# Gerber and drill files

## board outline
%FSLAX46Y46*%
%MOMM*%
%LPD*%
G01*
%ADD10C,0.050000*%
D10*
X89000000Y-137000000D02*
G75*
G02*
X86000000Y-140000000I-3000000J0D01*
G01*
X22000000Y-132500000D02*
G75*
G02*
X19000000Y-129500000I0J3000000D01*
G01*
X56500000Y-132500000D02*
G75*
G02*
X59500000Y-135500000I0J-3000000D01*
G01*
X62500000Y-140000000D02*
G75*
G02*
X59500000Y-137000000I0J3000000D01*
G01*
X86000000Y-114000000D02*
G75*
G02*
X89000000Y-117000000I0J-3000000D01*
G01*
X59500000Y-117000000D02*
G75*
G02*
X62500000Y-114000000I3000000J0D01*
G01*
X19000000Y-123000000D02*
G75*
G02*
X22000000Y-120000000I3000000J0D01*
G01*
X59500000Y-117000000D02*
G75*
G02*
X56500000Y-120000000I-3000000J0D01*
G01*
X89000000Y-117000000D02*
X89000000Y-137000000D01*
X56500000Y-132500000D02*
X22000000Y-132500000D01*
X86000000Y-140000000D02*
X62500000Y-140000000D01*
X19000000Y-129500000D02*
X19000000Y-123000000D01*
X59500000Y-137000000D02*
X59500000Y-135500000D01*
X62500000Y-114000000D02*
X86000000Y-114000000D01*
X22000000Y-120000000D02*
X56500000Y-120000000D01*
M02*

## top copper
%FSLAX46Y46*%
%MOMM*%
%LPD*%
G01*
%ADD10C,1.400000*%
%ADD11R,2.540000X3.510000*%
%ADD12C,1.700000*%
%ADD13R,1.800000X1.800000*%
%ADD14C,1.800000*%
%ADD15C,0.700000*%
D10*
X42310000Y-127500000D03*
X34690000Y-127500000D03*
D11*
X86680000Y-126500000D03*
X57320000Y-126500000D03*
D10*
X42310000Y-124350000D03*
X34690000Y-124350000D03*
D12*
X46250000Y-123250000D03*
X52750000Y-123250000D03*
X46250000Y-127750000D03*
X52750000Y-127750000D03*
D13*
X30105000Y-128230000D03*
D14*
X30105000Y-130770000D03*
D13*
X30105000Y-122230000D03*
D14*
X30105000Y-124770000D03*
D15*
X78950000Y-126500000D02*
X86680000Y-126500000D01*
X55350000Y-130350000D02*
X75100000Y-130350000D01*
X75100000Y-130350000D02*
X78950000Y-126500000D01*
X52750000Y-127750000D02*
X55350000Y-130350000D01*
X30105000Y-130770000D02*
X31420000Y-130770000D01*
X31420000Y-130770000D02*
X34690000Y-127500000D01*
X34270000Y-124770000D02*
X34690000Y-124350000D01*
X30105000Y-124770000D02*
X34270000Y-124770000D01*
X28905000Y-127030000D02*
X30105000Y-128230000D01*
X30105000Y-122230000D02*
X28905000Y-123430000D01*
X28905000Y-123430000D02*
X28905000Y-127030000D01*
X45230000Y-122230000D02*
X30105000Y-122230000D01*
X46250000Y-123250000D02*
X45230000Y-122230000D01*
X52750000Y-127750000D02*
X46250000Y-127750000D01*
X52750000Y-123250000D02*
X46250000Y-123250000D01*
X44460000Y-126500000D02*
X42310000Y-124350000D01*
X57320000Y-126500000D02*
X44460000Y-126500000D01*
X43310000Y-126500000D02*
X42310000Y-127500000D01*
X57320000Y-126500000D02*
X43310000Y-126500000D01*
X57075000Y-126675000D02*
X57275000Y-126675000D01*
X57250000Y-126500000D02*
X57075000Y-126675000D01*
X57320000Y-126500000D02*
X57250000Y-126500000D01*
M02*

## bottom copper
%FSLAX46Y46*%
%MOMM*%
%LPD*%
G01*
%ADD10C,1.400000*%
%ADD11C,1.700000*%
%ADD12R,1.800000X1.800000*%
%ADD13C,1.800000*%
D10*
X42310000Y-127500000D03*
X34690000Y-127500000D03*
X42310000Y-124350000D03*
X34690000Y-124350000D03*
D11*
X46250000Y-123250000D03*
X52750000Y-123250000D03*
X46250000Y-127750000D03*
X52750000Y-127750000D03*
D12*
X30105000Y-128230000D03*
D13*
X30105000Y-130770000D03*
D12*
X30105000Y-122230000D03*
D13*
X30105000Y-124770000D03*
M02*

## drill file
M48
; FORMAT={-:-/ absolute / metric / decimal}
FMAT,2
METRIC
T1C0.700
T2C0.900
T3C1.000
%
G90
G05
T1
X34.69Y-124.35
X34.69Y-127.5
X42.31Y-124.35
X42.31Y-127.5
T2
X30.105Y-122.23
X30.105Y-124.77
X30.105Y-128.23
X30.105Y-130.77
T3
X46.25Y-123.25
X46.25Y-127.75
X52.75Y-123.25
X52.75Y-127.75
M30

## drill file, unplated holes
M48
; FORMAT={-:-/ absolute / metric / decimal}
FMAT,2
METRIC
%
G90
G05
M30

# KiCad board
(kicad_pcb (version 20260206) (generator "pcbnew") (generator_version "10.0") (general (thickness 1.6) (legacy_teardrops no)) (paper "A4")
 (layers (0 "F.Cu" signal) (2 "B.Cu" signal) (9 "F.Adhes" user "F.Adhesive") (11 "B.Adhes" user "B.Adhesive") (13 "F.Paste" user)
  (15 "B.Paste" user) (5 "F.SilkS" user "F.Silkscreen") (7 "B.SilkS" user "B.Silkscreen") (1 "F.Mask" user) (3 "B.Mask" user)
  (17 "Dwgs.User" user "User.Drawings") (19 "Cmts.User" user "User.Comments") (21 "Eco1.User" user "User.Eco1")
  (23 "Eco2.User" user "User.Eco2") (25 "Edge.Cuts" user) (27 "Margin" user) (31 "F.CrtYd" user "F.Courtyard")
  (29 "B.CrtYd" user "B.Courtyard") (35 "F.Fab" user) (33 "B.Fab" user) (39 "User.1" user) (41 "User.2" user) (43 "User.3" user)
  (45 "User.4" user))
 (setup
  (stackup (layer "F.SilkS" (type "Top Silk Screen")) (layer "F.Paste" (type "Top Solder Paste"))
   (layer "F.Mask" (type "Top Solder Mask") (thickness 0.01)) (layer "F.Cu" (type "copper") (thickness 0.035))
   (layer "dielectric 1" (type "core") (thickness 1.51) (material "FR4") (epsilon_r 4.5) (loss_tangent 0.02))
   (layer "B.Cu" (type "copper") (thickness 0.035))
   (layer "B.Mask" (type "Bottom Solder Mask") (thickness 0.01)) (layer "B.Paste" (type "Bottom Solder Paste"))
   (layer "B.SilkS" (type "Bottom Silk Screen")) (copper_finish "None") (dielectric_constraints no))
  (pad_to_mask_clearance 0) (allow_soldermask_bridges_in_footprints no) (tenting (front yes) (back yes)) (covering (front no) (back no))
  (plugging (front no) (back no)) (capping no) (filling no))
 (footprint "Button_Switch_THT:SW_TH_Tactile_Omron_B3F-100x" (layer "F.Cu") (at 46.25 123.25)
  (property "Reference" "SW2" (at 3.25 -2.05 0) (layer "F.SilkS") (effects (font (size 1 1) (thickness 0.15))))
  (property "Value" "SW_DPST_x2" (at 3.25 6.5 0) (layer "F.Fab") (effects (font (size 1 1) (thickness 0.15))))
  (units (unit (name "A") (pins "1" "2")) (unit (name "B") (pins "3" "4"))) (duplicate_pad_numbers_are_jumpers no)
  (pad "1" thru_hole circle (at 0 0) (size 1.7 1.7) (drill 1) (layers "*.Cu" "*.Mask") (remove_unused_layers no) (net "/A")
   (thermal_bridge_angle 90))
  (pad "1" thru_hole circle (at 6.5 0) (size 1.7 1.7) (drill 1) (layers "*.Cu" "*.Mask") (remove_unused_layers no) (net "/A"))
  (pad "2" thru_hole circle (at 0 4.5) (size 1.7 1.7) (drill 1) (layers "*.Cu" "*.Mask") (remove_unused_layers no) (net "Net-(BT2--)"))
  (pad "2" thru_hole circle (at 6.5 4.5) (size 1.7 1.7) (drill 1) (layers "*.Cu" "*.Mask") (remove_unused_layers no) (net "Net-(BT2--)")))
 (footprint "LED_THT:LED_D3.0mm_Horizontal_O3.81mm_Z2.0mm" (layer "F.Cu") (at 30.105 122.23 -90)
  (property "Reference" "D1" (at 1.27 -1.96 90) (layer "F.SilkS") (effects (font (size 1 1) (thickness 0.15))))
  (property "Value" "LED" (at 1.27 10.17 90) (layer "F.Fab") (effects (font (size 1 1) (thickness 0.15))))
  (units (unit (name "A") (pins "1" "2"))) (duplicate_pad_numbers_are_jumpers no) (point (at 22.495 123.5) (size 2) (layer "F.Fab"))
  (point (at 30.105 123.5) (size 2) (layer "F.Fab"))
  (pad "1" thru_hole rect (at 0 0 270) (size 1.8 1.8) (drill 0.9) (layers "*.Cu" "*.Mask") (remove_unused_layers no) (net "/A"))
  (pad "2" thru_hole circle (at 2.54 0 270) (size 1.8 1.8) (drill 0.9) (layers "*.Cu" "*.Mask") (remove_unused_layers no) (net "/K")))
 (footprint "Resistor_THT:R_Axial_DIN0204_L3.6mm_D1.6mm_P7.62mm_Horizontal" (layer "F.Cu") (at 42.31 127.5 180)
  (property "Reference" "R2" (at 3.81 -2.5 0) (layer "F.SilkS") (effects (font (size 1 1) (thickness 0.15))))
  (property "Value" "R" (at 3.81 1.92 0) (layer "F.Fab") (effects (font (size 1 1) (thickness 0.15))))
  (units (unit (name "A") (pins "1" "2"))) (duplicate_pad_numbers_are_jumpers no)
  (pad "1" thru_hole circle (at 0 0 180) (size 1.4 1.4) (drill 0.7) (layers "*.Cu" "*.Mask") (remove_unused_layers no) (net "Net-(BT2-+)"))
  (pad "2" thru_hole circle (at 7.62 0 180) (size 1.4 1.4) (drill 0.7) (layers "*.Cu" "*.Mask") (remove_unused_layers no) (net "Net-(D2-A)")))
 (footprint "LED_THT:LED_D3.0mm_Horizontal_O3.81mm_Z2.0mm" (layer "F.Cu") (at 30.105 128.23 -90)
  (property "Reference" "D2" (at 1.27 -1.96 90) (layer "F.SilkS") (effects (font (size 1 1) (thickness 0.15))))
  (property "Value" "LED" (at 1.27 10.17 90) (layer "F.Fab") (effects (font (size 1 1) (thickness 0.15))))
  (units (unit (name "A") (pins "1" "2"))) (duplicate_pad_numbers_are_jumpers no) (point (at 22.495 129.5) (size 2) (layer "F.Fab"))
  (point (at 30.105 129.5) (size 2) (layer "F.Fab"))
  (pad "1" thru_hole rect (at 0 0 270) (size 1.8 1.8) (drill 0.9) (layers "*.Cu" "*.Mask") (remove_unused_layers no) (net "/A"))
  (pad "2" thru_hole circle (at 2.54 0 270) (size 1.8 1.8) (drill 0.9) (layers "*.Cu" "*.Mask") (remove_unused_layers no) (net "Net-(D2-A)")))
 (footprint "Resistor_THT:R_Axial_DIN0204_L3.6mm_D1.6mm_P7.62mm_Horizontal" (layer "F.Cu") (at 34.69 124.35)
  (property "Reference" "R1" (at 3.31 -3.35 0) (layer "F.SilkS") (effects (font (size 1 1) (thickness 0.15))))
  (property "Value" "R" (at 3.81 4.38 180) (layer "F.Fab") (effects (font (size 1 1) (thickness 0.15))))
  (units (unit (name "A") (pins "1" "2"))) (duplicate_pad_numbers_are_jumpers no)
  (pad "1" thru_hole circle (at 0 0) (size 1.4 1.4) (drill 0.7) (layers "*.Cu" "*.Mask") (remove_unused_layers no) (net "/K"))
  (pad "2" thru_hole circle (at 7.62 0) (size 1.4 1.4) (drill 0.7) (layers "*.Cu" "*.Mask") (remove_unused_layers no) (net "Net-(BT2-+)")))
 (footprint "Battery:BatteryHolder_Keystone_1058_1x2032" (layer "F.Cu") (at 72 126.5)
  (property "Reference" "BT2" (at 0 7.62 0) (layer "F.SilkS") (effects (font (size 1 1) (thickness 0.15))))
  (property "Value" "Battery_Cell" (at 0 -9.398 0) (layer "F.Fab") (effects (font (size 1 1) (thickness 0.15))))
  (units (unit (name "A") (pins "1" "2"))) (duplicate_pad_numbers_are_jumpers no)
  (pad "1" smd rect (at -14.68 0) (size 2.54 3.51) (layers "F.Cu" "F.Mask" "F.Paste") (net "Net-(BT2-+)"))
  (pad "2" smd rect (at 14.68 0) (size 2.54 3.51) (layers "F.Cu" "F.Mask" "F.Paste") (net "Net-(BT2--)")))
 (gr_arc (start 19 123) (mid 19.87868 120.87868) (end 22 120) (stroke (width 0.05) (type default)) (layer "Edge.Cuts"))
 (gr_line (start 19 129.5) (end 19 123) (stroke (width 0.05) (type default)) (layer "Edge.Cuts"))
 (gr_line (start 22 120) (end 56.5 120) (stroke (width 0.05) (type default)) (layer "Edge.Cuts"))
 (gr_arc (start 22 132.5) (mid 19.87868 131.62132) (end 19 129.5) (stroke (width 0.05) (type default)) (layer "Edge.Cuts"))
 (gr_line (start 56.5 132.5) (end 22 132.5) (stroke (width 0.05) (type default)) (layer "Edge.Cuts"))
 (gr_arc (start 56.5 132.5) (mid 58.62132 133.37868) (end 59.5 135.5) (stroke (width 0.05) (type default)) (layer "Edge.Cuts"))
 (gr_arc (start 59.5 117) (mid 58.62132 119.12132) (end 56.5 120) (stroke (width 0.05) (type default)) (layer "Edge.Cuts"))
 (gr_arc (start 59.5 117) (mid 60.37868 114.87868) (end 62.5 114) (stroke (width 0.05) (type default)) (layer "Edge.Cuts"))
 (gr_line (start 59.5 137) (end 59.5 135.5) (stroke (width 0.05) (type default)) (layer "Edge.Cuts"))
 (gr_line (start 62.5 114) (end 86 114) (stroke (width 0.05) (type default)) (layer "Edge.Cuts"))
 (gr_arc (start 62.5 140) (mid 60.37868 139.12132) (end 59.5 137) (stroke (width 0.05) (type default)) (layer "Edge.Cuts"))
 (gr_arc (start 86 114) (mid 88.12132 114.87868) (end 89 117) (stroke (width 0.05) (type default)) (layer "Edge.Cuts"))
 (gr_line (start 86 140) (end 62.5 140) (stroke (width 0.05) (type default)) (layer "Edge.Cuts"))
 (gr_line (start 89 117) (end 89 137) (stroke (width 0.05) (type default)) (layer "Edge.Cuts"))
 (gr_arc (start 89 137) (mid 88.12132 139.12132) (end 86 140) (stroke (width 0.05) (type default)) (layer "Edge.Cuts"))
 (segment (start 28.905 127.03) (end 30.105 128.23) (width 0.7) (layer "F.Cu") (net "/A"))
 (segment (start 30.105 122.23) (end 28.905 123.43) (width 0.7) (layer "F.Cu") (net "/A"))
 (segment (start 46.25 123.25) (end 45.23 122.23) (width 0.7) (layer "F.Cu") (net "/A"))
 (segment (start 45.23 122.23) (end 30.105 122.23) (width 0.7) (layer "F.Cu") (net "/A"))
 (segment (start 52.75 123.25) (end 46.25 123.25) (width 0.7) (layer "F.Cu") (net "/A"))
 (segment (start 28.905 123.43) (end 28.905 127.03) (width 0.7) (layer "F.Cu") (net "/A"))
 (segment (start 55.35 130.35) (end 75.1 130.35) (width 0.7) (layer "F.Cu") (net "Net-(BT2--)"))
 (segment (start 52.75 127.75) (end 55.35 130.35) (width 0.7) (layer "F.Cu") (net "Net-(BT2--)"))
 (segment (start 52.75 127.75) (end 46.25 127.75) (width 0.7) (layer "F.Cu") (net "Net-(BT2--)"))
 (segment (start 78.95 126.5) (end 86.68 126.5) (width 0.7) (layer "F.Cu") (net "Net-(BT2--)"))
 (segment (start 75.1 130.35) (end 78.95 126.5) (width 0.7) (layer "F.Cu") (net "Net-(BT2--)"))
 (segment (start 34.27 124.77) (end 34.69 124.35) (width 0.7) (layer "F.Cu") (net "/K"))
 (segment (start 30.105 124.77) (end 34.27 124.77) (width 0.7) (layer "F.Cu") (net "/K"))
 (segment (start 57.32 126.5) (end 43.31 126.5) (width 0.7) (layer "F.Cu") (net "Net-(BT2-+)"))
 (segment (start 57.32 126.5) (end 57.25 126.5) (width 0.7) (layer "F.Cu") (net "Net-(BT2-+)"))
 (segment (start 44.46 126.5) (end 42.31 124.35) (width 0.7) (layer "F.Cu") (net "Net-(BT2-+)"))
 (segment (start 57.32 126.5) (end 44.46 126.5) (width 0.7) (layer "F.Cu") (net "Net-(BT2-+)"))
 (segment (start 43.31 126.5) (end 42.31 127.5) (width 0.7) (layer "F.Cu") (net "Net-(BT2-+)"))
 (segment (start 57.075 126.675) (end 57.275 126.675) (width 0.7) (layer "F.Cu") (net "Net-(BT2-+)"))
 (segment (start 57.25 126.5) (end 57.075 126.675) (width 0.7) (layer "F.Cu") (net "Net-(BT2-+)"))
 (segment (start 30.105 130.77) (end 31.42 130.77) (width 0.7) (layer "F.Cu") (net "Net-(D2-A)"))
 (segment (start 31.42 130.77) (end 34.69 127.5) (width 0.7) (layer "F.Cu") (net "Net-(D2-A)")))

